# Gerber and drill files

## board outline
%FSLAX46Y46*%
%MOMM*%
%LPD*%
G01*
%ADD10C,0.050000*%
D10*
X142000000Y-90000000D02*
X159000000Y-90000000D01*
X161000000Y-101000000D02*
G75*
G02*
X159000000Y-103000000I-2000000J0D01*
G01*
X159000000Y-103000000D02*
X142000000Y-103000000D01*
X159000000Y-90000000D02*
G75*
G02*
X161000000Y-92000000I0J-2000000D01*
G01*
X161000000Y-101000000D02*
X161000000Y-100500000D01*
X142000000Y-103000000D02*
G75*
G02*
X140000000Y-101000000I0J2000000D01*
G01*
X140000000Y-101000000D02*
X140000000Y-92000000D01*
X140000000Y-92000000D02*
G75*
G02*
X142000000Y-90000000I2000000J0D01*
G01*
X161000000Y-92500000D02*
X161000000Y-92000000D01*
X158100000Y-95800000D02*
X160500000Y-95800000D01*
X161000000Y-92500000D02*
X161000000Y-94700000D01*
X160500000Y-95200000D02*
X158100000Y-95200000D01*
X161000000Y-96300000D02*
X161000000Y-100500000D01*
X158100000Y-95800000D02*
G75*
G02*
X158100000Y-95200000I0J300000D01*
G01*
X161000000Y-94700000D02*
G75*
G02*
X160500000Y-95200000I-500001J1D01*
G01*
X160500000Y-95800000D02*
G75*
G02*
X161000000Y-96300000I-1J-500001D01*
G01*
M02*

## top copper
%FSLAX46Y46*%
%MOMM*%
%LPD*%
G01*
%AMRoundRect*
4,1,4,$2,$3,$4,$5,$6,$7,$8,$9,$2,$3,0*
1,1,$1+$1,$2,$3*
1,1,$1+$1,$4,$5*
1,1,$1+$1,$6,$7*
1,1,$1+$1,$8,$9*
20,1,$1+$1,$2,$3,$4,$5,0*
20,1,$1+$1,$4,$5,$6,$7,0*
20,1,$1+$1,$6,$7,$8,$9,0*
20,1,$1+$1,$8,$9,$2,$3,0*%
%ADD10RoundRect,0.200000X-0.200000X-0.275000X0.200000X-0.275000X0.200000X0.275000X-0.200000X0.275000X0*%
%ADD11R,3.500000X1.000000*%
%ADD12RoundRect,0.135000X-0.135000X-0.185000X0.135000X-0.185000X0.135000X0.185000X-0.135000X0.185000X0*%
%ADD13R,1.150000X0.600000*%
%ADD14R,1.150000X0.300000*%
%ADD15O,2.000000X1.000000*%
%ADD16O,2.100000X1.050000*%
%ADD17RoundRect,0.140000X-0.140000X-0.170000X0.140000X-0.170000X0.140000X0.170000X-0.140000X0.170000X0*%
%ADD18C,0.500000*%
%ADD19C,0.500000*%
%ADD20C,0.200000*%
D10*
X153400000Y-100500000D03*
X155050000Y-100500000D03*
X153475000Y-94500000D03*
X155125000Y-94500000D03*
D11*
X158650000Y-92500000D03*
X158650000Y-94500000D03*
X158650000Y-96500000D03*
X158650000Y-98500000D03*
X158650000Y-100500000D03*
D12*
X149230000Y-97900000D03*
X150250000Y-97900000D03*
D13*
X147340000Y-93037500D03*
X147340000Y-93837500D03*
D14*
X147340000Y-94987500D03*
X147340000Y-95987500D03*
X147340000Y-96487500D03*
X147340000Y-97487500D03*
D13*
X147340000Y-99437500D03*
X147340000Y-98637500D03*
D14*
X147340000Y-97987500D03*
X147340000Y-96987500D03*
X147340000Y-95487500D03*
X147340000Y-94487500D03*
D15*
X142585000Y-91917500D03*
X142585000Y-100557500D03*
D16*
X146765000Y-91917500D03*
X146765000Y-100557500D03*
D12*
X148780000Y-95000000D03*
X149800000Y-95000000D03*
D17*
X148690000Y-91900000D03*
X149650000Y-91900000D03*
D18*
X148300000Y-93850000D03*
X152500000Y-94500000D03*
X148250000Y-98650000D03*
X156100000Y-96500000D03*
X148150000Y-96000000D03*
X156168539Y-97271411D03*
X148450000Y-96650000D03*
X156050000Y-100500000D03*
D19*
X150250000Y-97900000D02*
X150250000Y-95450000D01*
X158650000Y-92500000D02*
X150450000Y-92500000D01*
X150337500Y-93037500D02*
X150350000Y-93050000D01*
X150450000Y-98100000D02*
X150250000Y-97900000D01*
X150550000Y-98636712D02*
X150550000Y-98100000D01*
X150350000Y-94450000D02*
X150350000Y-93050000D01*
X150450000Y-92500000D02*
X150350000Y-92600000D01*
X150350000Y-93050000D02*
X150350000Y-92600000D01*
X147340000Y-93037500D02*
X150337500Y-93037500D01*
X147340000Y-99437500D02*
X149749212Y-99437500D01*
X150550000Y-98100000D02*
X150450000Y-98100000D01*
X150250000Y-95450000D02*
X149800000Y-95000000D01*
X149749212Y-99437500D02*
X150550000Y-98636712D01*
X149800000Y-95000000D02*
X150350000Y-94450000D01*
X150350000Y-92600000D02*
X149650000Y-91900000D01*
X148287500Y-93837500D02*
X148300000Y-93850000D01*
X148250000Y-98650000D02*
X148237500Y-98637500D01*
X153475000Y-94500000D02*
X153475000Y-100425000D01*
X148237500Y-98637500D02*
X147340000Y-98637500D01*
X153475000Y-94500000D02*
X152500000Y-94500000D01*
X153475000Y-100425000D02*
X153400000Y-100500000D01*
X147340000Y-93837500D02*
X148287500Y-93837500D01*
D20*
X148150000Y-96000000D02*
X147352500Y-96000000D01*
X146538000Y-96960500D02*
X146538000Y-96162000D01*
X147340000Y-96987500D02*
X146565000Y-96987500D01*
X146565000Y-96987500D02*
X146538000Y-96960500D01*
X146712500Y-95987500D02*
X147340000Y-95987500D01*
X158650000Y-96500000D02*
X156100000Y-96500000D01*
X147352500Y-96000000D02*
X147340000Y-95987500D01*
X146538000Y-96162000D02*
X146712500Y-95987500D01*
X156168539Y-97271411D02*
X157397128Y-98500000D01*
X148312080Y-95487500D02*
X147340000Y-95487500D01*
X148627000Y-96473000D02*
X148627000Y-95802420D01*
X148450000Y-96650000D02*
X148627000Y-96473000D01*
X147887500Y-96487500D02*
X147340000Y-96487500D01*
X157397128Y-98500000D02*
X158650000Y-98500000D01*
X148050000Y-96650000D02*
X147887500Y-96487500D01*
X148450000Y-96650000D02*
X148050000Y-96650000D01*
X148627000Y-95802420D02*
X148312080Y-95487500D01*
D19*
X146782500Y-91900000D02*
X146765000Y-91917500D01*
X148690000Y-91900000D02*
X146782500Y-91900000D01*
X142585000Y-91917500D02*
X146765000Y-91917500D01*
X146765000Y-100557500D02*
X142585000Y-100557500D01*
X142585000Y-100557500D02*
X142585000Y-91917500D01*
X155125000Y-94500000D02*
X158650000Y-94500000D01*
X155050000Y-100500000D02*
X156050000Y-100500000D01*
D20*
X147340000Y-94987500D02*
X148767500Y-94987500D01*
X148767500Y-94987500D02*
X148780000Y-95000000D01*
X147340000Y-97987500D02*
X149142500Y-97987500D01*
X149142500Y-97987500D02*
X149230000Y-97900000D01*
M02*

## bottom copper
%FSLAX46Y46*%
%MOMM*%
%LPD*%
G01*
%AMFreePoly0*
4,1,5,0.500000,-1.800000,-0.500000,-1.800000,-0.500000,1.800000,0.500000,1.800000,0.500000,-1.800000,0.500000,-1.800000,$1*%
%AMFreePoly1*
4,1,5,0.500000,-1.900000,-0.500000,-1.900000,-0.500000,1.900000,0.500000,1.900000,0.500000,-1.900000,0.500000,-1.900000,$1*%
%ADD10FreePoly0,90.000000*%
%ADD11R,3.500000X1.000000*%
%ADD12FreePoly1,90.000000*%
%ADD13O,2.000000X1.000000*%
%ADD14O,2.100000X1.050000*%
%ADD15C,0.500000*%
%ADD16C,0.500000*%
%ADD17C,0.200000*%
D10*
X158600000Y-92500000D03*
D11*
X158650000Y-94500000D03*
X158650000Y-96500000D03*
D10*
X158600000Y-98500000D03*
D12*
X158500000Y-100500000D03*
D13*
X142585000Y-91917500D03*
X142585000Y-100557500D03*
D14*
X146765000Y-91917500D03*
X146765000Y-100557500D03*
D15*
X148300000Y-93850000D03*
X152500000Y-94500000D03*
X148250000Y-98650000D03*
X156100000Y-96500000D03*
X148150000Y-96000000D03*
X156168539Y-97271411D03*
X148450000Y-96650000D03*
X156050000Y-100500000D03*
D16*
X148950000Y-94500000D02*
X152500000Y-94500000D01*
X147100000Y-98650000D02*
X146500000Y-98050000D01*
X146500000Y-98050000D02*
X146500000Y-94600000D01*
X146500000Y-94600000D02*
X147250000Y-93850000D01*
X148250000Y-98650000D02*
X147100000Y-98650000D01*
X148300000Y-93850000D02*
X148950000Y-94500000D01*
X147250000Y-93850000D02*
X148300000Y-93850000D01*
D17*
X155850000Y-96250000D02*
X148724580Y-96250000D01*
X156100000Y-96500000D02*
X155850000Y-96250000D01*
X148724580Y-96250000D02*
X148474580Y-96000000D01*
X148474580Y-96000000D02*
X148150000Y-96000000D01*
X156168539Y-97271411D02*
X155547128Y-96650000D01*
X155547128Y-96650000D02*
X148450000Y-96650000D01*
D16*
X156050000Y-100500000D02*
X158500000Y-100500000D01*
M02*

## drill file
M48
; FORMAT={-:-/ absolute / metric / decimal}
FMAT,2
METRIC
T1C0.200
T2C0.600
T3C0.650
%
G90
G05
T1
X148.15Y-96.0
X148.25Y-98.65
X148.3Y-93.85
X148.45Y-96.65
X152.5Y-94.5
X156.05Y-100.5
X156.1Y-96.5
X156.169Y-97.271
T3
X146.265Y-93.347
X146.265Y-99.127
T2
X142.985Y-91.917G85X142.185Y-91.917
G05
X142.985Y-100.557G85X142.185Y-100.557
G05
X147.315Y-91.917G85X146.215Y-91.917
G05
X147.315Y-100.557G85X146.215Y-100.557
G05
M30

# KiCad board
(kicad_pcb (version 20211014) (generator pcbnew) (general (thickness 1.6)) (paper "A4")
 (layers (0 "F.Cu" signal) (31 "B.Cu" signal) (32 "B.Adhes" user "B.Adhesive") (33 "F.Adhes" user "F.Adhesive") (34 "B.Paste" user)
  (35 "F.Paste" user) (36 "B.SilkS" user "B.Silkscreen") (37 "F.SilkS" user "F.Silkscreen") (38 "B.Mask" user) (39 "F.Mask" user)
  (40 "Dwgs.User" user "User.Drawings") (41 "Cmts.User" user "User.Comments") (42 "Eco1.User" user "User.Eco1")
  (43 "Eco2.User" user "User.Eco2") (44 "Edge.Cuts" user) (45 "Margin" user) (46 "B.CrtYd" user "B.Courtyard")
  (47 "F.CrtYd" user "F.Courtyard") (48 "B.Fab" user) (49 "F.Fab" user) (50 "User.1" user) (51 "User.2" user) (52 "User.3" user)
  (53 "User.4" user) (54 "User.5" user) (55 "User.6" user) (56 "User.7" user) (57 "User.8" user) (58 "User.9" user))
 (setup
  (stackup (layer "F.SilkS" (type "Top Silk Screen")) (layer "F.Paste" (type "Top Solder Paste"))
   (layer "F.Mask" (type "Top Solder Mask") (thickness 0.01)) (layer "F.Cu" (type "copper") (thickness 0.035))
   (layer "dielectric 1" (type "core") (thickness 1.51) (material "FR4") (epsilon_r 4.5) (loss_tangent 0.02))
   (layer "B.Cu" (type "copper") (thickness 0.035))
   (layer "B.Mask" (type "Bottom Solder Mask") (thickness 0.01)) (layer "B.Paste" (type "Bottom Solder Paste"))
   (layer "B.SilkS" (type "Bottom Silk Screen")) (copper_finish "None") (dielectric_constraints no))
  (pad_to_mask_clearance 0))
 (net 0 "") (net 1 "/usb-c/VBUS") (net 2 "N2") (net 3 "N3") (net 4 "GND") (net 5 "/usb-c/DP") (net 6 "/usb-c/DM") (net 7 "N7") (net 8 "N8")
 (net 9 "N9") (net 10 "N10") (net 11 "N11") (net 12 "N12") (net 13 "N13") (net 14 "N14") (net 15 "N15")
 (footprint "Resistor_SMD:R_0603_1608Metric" (layer "F.Cu") (at 154.225 100.5)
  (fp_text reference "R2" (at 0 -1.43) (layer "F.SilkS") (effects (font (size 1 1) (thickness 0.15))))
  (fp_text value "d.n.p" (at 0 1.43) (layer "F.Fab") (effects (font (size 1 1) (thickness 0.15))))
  (pad "1" smd roundrect (at -0.825 0) (size 0.8 0.95) (layers "F.Cu" "F.Paste" "F.Mask") (roundrect_rratio 0.25) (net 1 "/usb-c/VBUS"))
  (pad "2" smd roundrect (at 0.825 0) (size 0.8 0.95) (layers "F.Cu" "F.Paste" "F.Mask") (roundrect_rratio 0.25) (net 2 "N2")))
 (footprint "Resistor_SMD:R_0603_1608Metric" (layer "F.Cu") (at 154.3 94.5)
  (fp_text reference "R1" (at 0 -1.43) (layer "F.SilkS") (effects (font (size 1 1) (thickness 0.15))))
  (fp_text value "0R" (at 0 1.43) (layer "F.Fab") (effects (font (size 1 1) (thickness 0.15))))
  (pad "1" smd roundrect (at -0.825 0) (size 0.8 0.95) (layers "F.Cu" "F.Paste" "F.Mask") (roundrect_rratio 0.25) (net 1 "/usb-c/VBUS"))
  (pad "2" smd roundrect (at 0.825 0) (size 0.8 0.95) (layers "F.Cu" "F.Paste" "F.Mask") (roundrect_rratio 0.25) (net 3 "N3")))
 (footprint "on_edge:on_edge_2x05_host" (layer "F.Cu") (at 161 96.5 -90)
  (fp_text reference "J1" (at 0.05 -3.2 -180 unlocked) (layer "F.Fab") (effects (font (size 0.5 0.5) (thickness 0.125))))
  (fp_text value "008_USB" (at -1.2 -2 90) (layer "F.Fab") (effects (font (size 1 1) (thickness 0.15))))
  (fp_line (start -0.7 2.9) (end -0.7 0.5) (layer "Edge.Cuts") (width 0.05))
  (fp_line (start -4 0) (end -1.8 0) (layer "Edge.Cuts") (width 0.05))
  (fp_line (start -1.3 0.5) (end -1.3 2.9) (layer "Edge.Cuts") (width 0.05))
  (fp_line (start -0.2 0) (end 4 0) (layer "Edge.Cuts") (width 0.05))
  (fp_arc (start -0.7 2.9) (mid -1 3.2) (end -1.3 2.9) (layer "Edge.Cuts") (width 0.05))
  (fp_arc (start -1.8 0) (mid -1.446447 0.146447) (end -1.3 0.5) (layer "Edge.Cuts") (width 0.05))
  (fp_arc (start -0.7 0.5) (mid -0.553553 0.146447) (end -0.2 0) (layer "Edge.Cuts") (width 0.05))
  (pad "1" smd rect (at -4 2.35 270) (size 1 3.5) (layers "F.Cu" "F.Mask") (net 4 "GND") (zone_connect 0))
  (pad "2" smd rect (at -2 2.35 270) (size 1 3.5) (layers "F.Cu" "F.Mask") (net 3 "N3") (zone_connect 0))
  (pad "3" smd rect (at 0 2.35 270) (size 1 3.5) (layers "F.Cu" "F.Mask") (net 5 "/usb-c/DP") (zone_connect 0))
  (pad "4" smd rect (at 2 2.35 270) (size 1 3.5) (layers "F.Cu" "F.Mask") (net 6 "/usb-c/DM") (zone_connect 0))
  (pad "5" smd rect (at 4 2.35 270) (size 1 3.5) (layers "F.Cu" "F.Mask") (zone_connect 0))
  (pad "6" smd custom (at -4 2.4 90) (size 1 3.6) (layers "B.Cu" "B.Mask") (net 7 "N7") (zone_connect 0)
   (options (clearance outline) (anchor rect)) (primitives))
  (pad "7" smd rect (at -2 2.35 90) (size 1 3.5) (layers "B.Cu" "B.Mask") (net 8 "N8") (zone_connect 0))
  (pad "8" smd rect (at 0 2.35 90) (size 1 3.5) (layers "B.Cu" "B.Mask") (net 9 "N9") (zone_connect 0))
  (pad "9" smd custom (at 2 2.4 90) (size 1 3.6) (layers "B.Cu" "B.Mask") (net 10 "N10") (zone_connect 0)
   (options (clearance outline) (anchor rect)) (primitives))
  (pad "10" smd custom (at 4 2.5 90) (size 1 3.8) (layers "B.Cu" "B.Mask") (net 2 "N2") (zone_connect 0)
   (options (clearance outline) (anchor rect)) (primitives))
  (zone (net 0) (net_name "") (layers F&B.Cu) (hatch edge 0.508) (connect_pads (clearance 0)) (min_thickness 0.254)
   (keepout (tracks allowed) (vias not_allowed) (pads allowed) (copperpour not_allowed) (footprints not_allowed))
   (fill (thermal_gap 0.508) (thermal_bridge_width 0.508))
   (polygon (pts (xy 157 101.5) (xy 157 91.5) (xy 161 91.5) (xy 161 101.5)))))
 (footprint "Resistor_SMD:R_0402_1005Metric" (layer "F.Cu") (at 149.74 97.9)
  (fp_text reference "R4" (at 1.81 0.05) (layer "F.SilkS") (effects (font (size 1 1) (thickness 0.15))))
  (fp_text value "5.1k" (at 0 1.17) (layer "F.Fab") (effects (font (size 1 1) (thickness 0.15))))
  (pad "1" smd roundrect (at -0.51 0) (size 0.54 0.64) (layers "F.Cu" "F.Paste" "F.Mask") (roundrect_rratio 0.25) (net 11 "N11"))
  (pad "2" smd roundrect (at 0.51 0) (size 0.54 0.64) (layers "F.Cu" "F.Paste" "F.Mask") (roundrect_rratio 0.25) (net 4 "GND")))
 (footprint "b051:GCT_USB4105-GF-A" (layer "F.Cu") (at 142.585 96.2375 -90)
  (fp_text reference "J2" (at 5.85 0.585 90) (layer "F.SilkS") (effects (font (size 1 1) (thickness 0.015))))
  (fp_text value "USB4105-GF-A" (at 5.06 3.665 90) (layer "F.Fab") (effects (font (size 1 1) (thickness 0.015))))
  (pad "" np_thru_hole circle (at 2.89 -3.68 270) (size 0.65 0.65) (drill 0.65) (layers *.Cu *.Mask))
  (pad "" np_thru_hole circle (at -2.89 -3.68 270) (size 0.65 0.65) (drill 0.65) (layers *.Cu *.Mask))
  (pad "A1/B12" smd rect (at -3.2 -4.755 270) (size 0.6 1.15) (layers "F.Cu" "F.Paste" "F.Mask") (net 4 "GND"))
  (pad "A4/B9" smd rect (at -2.4 -4.755 270) (size 0.6 1.15) (layers "F.Cu" "F.Paste" "F.Mask") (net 1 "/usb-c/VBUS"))
  (pad "A5" smd rect (at -1.25 -4.755 270) (size 0.3 1.15) (layers "F.Cu" "F.Paste" "F.Mask") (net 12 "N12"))
  (pad "A6" smd rect (at -0.25 -4.755 270) (size 0.3 1.15) (layers "F.Cu" "F.Paste" "F.Mask") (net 5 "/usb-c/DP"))
  (pad "A7" smd rect (at 0.25 -4.755 270) (size 0.3 1.15) (layers "F.Cu" "F.Paste" "F.Mask") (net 6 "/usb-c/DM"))
  (pad "A8" smd rect (at 1.25 -4.755 270) (size 0.3 1.15) (layers "F.Cu" "F.Paste" "F.Mask") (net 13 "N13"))
  (pad "B1/A12" smd rect (at 3.2 -4.755 270) (size 0.6 1.15) (layers "F.Cu" "F.Paste" "F.Mask") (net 4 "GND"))
  (pad "B4/A9" smd rect (at 2.4 -4.755 270) (size 0.6 1.15) (layers "F.Cu" "F.Paste" "F.Mask") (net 1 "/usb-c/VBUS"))
  (pad "B5" smd rect (at 1.75 -4.755 270) (size 0.3 1.15) (layers "F.Cu" "F.Paste" "F.Mask") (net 11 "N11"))
  (pad "B6" smd rect (at 0.75 -4.755 270) (size 0.3 1.15) (layers "F.Cu" "F.Paste" "F.Mask") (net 5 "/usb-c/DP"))
  (pad "B7" smd rect (at -0.75 -4.755 270) (size 0.3 1.15) (layers "F.Cu" "F.Paste" "F.Mask") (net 6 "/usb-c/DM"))
  (pad "B8" smd rect (at -1.75 -4.755 270) (size 0.3 1.15) (layers "F.Cu" "F.Paste" "F.Mask") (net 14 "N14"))
  (pad "G1" thru_hole oval (at -4.32 0 270) (size 1 2) (drill oval 0.6 1.4) (layers *.Cu *.Mask) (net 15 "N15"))
  (pad "G2" thru_hole oval (at 4.32 0 270) (size 1 2) (drill oval 0.6 1.4) (layers *.Cu *.Mask) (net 15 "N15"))
  (pad "G3" thru_hole oval (at -4.32 -4.18 270) (size 1.05 2.1) (drill oval 0.6 1.7) (layers *.Cu *.Mask) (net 15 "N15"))
  (pad "G4" thru_hole oval (at 4.32 -4.18 270) (size 1.05 2.1) (drill oval 0.6 1.7) (layers *.Cu *.Mask) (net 15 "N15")))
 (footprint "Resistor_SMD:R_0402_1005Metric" (layer "F.Cu") (at 149.29 95)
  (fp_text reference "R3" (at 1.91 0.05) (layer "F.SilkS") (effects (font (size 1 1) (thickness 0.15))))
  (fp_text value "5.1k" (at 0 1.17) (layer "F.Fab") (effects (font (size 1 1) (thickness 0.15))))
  (pad "1" smd roundrect (at -0.51 0) (size 0.54 0.64) (layers "F.Cu" "F.Paste" "F.Mask") (roundrect_rratio 0.25) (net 12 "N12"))
  (pad "2" smd roundrect (at 0.51 0) (size 0.54 0.64) (layers "F.Cu" "F.Paste" "F.Mask") (roundrect_rratio 0.25) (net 4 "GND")))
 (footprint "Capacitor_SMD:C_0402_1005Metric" (layer "F.Cu") (at 149.17 91.9)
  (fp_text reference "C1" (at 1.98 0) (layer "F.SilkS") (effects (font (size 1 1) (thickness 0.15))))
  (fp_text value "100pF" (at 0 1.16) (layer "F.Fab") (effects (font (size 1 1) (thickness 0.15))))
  (pad "1" smd roundrect (at -0.48 0) (size 0.56 0.62) (layers "F.Cu" "F.Paste" "F.Mask") (roundrect_rratio 0.25) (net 15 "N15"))
  (pad "2" smd roundrect (at 0.48 0) (size 0.56 0.62) (layers "F.Cu" "F.Paste" "F.Mask") (roundrect_rratio 0.25) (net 4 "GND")))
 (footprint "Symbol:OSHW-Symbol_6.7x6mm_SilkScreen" (layer "B.Cu") (at 151.75 99.8 180)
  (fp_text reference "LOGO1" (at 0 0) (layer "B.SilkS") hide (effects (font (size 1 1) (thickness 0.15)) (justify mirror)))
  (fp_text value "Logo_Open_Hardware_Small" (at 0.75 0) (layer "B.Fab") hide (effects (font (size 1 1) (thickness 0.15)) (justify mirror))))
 (gr_line (start 142 90) (end 159 90) (layer "Edge.Cuts") (width 0.05))
 (gr_arc (start 161 101) (mid 160.414214 102.414214) (end 159 103) (layer "Edge.Cuts") (width 0.05))
 (gr_line (start 159 103) (end 142 103) (layer "Edge.Cuts") (width 0.05))
 (gr_arc (start 159 90) (mid 160.414214 90.585786) (end 161 92) (layer "Edge.Cuts") (width 0.05))
 (gr_line (start 161 101) (end 161 100.5) (layer "Edge.Cuts") (width 0.05))
 (gr_arc (start 142 103) (mid 140.585786 102.414214) (end 140 101) (layer "Edge.Cuts") (width 0.05))
 (gr_line (start 140 101) (end 140 92) (layer "Edge.Cuts") (width 0.05))
 (gr_arc (start 140 92) (mid 140.585786 90.585786) (end 142 90) (layer "Edge.Cuts") (width 0.05))
 (gr_line (start 161 92.5) (end 161 92) (layer "Edge.Cuts") (width 0.05))
 (segment (start 150.25 97.9) (end 150.25 95.45) (width 0.5) (layer "F.Cu") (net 4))
 (segment (start 158.65 92.5) (end 150.45 92.5) (width 0.5) (layer "F.Cu") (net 4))
 (segment (start 150.3375 93.0375) (end 150.35 93.05) (width 0.5) (layer "F.Cu") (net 4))
 (segment (start 150.45 98.1) (end 150.25 97.9) (width 0.5) (layer "F.Cu") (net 4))
 (segment (start 150.55 98.636712) (end 150.55 98.1) (width 0.5) (layer "F.Cu") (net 4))
 (segment (start 150.35 94.45) (end 150.35 93.05) (width 0.5) (layer "F.Cu") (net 4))
 (segment (start 150.45 92.5) (end 150.35 92.6) (width 0.5) (layer "F.Cu") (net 4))
 (segment (start 150.35 93.05) (end 150.35 92.6) (width 0.5) (layer "F.Cu") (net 4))
 (segment (start 147.34 93.0375) (end 150.3375 93.0375) (width 0.5) (layer "F.Cu") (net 4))
 (segment (start 147.34 99.4375) (end 149.749212 99.4375) (width 0.5) (layer "F.Cu") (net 4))
 (segment (start 150.55 98.1) (end 150.45 98.1) (width 0.5) (layer "F.Cu") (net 4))
 (segment (start 150.25 95.45) (end 149.8 95) (width 0.5) (layer "F.Cu") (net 4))
 (segment (start 149.749212 99.4375) (end 150.55 98.636712) (width 0.5) (layer "F.Cu") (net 4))
 (segment (start 149.8 95) (end 150.35 94.45) (width 0.5) (layer "F.Cu") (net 4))
 (segment (start 150.35 92.6) (end 149.65 91.9) (width 0.5) (layer "F.Cu") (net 4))
 (segment (start 148.2875 93.8375) (end 148.3 93.85) (width 0.5) (layer "F.Cu") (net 1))
 (segment (start 148.25 98.65) (end 148.2375 98.6375) (width 0.5) (layer "F.Cu") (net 1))
 (segment (start 153.475 94.5) (end 153.475 100.425) (width 0.5) (layer "F.Cu") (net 1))
 (segment (start 148.2375 98.6375) (end 147.34 98.6375) (width 0.5) (layer "F.Cu") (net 1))
 (segment (start 153.475 94.5) (end 152.5 94.5) (width 0.5) (layer "F.Cu") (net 1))
 (segment (start 153.475 100.425) (end 153.4 100.5) (width 0.5) (layer "F.Cu") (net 1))
 (segment (start 147.34 93.8375) (end 148.2875 93.8375) (width 0.5) (layer "F.Cu") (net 1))
 (via (at 148.3 93.85) (size 0.5) (drill 0.2) (layers "F.Cu" "B.Cu") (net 1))
 (via (at 152.5 94.5) (size 0.5) (drill 0.2) (layers "F.Cu" "B.Cu") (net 1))
 (via (at 148.25 98.65) (size 0.5) (drill 0.2) (layers "F.Cu" "B.Cu") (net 1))
 (segment (start 148.95 94.5) (end 152.5 94.5) (width 0.5) (layer "B.Cu") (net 1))
 (segment (start 147.1 98.65) (end 146.5 98.05) (width 0.5) (layer "B.Cu") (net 1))
 (segment (start 146.5 98.05) (end 146.5 94.6) (width 0.5) (layer "B.Cu") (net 1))
 (segment (start 146.5 94.6) (end 147.25 93.85) (width 0.5) (layer "B.Cu") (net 1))
 (segment (start 148.25 98.65) (end 147.1 98.65) (width 0.5) (layer "B.Cu") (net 1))
 (segment (start 148.3 93.85) (end 148.95 94.5) (width 0.5) (layer "B.Cu") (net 1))
 (segment (start 147.25 93.85) (end 148.3 93.85) (width 0.5) (layer "B.Cu") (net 1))
 (segment (start 148.15 96) (end 147.3525 96) (width 0.2) (layer "F.Cu") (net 5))
 (segment (start 146.538 96.9605) (end 146.538 96.162) (width 0.2) (layer "F.Cu") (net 5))
 (segment (start 147.34 96.9875) (end 146.565 96.9875) (width 0.2) (layer "F.Cu") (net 5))
 (segment (start 146.565 96.9875) (end 146.538 96.9605) (width 0.2) (layer "F.Cu") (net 5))
 (segment (start 146.7125 95.9875) (end 147.34 95.9875) (width 0.2) (layer "F.Cu") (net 5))
 (segment (start 158.65 96.5) (end 156.1 96.5) (width 0.2) (layer "F.Cu") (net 5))
 (segment (start 147.3525 96) (end 147.34 95.9875) (width 0.2) (layer "F.Cu") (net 5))
 (segment (start 146.538 96.162) (end 146.7125 95.9875) (width 0.2) (layer "F.Cu") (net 5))
 (via (at 156.1 96.5) (size 0.5) (drill 0.2) (layers "F.Cu" "B.Cu") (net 5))
 (via (at 148.15 96) (size 0.5) (drill 0.2) (layers "F.Cu" "B.Cu") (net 5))
 (segment (start 155.85 96.25) (end 148.72458 96.25) (width 0.2) (layer "B.Cu") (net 5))
 (segment (start 156.1 96.5) (end 155.85 96.25) (width 0.2) (layer "B.Cu") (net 5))
 (segment (start 148.72458 96.25) (end 148.47458 96) (width 0.2) (layer "B.Cu") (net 5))
 (segment (start 148.47458 96) (end 148.15 96) (width 0.2) (layer "B.Cu") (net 5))
 (segment (start 156.168539 97.271411) (end 157.397128 98.5) (width 0.2) (layer "F.Cu") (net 6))
 (segment (start 148.31208 95.4875) (end 147.34 95.4875) (width 0.2) (layer "F.Cu") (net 6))
 (segment (start 148.627 96.473) (end 148.627 95.80242) (width 0.2) (layer "F.Cu") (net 6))
 (segment (start 148.45 96.65) (end 148.627 96.473) (width 0.2) (layer "F.Cu") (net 6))
 (segment (start 147.8875 96.4875) (end 147.34 96.4875) (width 0.2) (layer "F.Cu") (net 6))
 (segment (start 157.397128 98.5) (end 158.65 98.5) (width 0.2) (layer "F.Cu") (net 6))
 (segment (start 148.05 96.65) (end 147.8875 96.4875) (width 0.2) (layer "F.Cu") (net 6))
 (segment (start 148.45 96.65) (end 148.05 96.65) (width 0.2) (layer "F.Cu") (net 6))
 (segment (start 148.627 95.80242) (end 148.31208 95.4875) (width 0.2) (layer "F.Cu") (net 6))
 (via (at 156.168539 97.271411) (size 0.5) (drill 0.2) (layers "F.Cu" "B.Cu") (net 6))
 (via (at 148.45 96.65) (size 0.5) (drill 0.2) (layers "F.Cu" "B.Cu") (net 6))
 (segment (start 156.168539 97.271411) (end 155.547128 96.65) (width 0.2) (layer "B.Cu") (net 6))
 (segment (start 155.547128 96.65) (end 148.45 96.65) (width 0.2) (layer "B.Cu") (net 6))
 (segment (start 146.7825 91.9) (end 146.765 91.9175) (width 0.5) (layer "F.Cu") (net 15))
 (segment (start 148.69 91.9) (end 146.7825 91.9) (width 0.5) (layer "F.Cu") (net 15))
 (segment (start 142.585 91.9175) (end 146.765 91.9175) (width 0.5) (layer "F.Cu") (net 15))
 (segment (start 146.765 100.5575) (end 142.585 100.5575) (width 0.5) (layer "F.Cu") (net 15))
 (segment (start 142.585 100.5575) (end 142.585 91.9175) (width 0.5) (layer "F.Cu") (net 15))
 (segment (start 155.125 94.5) (end 158.65 94.5) (width 0.5) (layer "F.Cu") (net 3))
 (segment (start 155.05 100.5) (end 156.05 100.5) (width 0.5) (layer "F.Cu") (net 2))
 (via (at 156.05 100.5) (size 0.5) (drill 0.2) (layers "F.Cu" "B.Cu") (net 2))
 (segment (start 156.05 100.5) (end 158.5 100.5) (width 0.5) (layer "B.Cu") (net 2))
 (segment (start 147.34 94.9875) (end 148.7675 94.9875) (width 0.2) (layer "F.Cu") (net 12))
 (segment (start 148.7675 94.9875) (end 148.78 95) (width 0.2) (layer "F.Cu") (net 12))
 (segment (start 147.34 97.9875) (end 149.1425 97.9875) (width 0.2) (layer "F.Cu") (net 11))
 (segment (start 149.1425 97.9875) (end 149.23 97.9) (width 0.2) (layer "F.Cu") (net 11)))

